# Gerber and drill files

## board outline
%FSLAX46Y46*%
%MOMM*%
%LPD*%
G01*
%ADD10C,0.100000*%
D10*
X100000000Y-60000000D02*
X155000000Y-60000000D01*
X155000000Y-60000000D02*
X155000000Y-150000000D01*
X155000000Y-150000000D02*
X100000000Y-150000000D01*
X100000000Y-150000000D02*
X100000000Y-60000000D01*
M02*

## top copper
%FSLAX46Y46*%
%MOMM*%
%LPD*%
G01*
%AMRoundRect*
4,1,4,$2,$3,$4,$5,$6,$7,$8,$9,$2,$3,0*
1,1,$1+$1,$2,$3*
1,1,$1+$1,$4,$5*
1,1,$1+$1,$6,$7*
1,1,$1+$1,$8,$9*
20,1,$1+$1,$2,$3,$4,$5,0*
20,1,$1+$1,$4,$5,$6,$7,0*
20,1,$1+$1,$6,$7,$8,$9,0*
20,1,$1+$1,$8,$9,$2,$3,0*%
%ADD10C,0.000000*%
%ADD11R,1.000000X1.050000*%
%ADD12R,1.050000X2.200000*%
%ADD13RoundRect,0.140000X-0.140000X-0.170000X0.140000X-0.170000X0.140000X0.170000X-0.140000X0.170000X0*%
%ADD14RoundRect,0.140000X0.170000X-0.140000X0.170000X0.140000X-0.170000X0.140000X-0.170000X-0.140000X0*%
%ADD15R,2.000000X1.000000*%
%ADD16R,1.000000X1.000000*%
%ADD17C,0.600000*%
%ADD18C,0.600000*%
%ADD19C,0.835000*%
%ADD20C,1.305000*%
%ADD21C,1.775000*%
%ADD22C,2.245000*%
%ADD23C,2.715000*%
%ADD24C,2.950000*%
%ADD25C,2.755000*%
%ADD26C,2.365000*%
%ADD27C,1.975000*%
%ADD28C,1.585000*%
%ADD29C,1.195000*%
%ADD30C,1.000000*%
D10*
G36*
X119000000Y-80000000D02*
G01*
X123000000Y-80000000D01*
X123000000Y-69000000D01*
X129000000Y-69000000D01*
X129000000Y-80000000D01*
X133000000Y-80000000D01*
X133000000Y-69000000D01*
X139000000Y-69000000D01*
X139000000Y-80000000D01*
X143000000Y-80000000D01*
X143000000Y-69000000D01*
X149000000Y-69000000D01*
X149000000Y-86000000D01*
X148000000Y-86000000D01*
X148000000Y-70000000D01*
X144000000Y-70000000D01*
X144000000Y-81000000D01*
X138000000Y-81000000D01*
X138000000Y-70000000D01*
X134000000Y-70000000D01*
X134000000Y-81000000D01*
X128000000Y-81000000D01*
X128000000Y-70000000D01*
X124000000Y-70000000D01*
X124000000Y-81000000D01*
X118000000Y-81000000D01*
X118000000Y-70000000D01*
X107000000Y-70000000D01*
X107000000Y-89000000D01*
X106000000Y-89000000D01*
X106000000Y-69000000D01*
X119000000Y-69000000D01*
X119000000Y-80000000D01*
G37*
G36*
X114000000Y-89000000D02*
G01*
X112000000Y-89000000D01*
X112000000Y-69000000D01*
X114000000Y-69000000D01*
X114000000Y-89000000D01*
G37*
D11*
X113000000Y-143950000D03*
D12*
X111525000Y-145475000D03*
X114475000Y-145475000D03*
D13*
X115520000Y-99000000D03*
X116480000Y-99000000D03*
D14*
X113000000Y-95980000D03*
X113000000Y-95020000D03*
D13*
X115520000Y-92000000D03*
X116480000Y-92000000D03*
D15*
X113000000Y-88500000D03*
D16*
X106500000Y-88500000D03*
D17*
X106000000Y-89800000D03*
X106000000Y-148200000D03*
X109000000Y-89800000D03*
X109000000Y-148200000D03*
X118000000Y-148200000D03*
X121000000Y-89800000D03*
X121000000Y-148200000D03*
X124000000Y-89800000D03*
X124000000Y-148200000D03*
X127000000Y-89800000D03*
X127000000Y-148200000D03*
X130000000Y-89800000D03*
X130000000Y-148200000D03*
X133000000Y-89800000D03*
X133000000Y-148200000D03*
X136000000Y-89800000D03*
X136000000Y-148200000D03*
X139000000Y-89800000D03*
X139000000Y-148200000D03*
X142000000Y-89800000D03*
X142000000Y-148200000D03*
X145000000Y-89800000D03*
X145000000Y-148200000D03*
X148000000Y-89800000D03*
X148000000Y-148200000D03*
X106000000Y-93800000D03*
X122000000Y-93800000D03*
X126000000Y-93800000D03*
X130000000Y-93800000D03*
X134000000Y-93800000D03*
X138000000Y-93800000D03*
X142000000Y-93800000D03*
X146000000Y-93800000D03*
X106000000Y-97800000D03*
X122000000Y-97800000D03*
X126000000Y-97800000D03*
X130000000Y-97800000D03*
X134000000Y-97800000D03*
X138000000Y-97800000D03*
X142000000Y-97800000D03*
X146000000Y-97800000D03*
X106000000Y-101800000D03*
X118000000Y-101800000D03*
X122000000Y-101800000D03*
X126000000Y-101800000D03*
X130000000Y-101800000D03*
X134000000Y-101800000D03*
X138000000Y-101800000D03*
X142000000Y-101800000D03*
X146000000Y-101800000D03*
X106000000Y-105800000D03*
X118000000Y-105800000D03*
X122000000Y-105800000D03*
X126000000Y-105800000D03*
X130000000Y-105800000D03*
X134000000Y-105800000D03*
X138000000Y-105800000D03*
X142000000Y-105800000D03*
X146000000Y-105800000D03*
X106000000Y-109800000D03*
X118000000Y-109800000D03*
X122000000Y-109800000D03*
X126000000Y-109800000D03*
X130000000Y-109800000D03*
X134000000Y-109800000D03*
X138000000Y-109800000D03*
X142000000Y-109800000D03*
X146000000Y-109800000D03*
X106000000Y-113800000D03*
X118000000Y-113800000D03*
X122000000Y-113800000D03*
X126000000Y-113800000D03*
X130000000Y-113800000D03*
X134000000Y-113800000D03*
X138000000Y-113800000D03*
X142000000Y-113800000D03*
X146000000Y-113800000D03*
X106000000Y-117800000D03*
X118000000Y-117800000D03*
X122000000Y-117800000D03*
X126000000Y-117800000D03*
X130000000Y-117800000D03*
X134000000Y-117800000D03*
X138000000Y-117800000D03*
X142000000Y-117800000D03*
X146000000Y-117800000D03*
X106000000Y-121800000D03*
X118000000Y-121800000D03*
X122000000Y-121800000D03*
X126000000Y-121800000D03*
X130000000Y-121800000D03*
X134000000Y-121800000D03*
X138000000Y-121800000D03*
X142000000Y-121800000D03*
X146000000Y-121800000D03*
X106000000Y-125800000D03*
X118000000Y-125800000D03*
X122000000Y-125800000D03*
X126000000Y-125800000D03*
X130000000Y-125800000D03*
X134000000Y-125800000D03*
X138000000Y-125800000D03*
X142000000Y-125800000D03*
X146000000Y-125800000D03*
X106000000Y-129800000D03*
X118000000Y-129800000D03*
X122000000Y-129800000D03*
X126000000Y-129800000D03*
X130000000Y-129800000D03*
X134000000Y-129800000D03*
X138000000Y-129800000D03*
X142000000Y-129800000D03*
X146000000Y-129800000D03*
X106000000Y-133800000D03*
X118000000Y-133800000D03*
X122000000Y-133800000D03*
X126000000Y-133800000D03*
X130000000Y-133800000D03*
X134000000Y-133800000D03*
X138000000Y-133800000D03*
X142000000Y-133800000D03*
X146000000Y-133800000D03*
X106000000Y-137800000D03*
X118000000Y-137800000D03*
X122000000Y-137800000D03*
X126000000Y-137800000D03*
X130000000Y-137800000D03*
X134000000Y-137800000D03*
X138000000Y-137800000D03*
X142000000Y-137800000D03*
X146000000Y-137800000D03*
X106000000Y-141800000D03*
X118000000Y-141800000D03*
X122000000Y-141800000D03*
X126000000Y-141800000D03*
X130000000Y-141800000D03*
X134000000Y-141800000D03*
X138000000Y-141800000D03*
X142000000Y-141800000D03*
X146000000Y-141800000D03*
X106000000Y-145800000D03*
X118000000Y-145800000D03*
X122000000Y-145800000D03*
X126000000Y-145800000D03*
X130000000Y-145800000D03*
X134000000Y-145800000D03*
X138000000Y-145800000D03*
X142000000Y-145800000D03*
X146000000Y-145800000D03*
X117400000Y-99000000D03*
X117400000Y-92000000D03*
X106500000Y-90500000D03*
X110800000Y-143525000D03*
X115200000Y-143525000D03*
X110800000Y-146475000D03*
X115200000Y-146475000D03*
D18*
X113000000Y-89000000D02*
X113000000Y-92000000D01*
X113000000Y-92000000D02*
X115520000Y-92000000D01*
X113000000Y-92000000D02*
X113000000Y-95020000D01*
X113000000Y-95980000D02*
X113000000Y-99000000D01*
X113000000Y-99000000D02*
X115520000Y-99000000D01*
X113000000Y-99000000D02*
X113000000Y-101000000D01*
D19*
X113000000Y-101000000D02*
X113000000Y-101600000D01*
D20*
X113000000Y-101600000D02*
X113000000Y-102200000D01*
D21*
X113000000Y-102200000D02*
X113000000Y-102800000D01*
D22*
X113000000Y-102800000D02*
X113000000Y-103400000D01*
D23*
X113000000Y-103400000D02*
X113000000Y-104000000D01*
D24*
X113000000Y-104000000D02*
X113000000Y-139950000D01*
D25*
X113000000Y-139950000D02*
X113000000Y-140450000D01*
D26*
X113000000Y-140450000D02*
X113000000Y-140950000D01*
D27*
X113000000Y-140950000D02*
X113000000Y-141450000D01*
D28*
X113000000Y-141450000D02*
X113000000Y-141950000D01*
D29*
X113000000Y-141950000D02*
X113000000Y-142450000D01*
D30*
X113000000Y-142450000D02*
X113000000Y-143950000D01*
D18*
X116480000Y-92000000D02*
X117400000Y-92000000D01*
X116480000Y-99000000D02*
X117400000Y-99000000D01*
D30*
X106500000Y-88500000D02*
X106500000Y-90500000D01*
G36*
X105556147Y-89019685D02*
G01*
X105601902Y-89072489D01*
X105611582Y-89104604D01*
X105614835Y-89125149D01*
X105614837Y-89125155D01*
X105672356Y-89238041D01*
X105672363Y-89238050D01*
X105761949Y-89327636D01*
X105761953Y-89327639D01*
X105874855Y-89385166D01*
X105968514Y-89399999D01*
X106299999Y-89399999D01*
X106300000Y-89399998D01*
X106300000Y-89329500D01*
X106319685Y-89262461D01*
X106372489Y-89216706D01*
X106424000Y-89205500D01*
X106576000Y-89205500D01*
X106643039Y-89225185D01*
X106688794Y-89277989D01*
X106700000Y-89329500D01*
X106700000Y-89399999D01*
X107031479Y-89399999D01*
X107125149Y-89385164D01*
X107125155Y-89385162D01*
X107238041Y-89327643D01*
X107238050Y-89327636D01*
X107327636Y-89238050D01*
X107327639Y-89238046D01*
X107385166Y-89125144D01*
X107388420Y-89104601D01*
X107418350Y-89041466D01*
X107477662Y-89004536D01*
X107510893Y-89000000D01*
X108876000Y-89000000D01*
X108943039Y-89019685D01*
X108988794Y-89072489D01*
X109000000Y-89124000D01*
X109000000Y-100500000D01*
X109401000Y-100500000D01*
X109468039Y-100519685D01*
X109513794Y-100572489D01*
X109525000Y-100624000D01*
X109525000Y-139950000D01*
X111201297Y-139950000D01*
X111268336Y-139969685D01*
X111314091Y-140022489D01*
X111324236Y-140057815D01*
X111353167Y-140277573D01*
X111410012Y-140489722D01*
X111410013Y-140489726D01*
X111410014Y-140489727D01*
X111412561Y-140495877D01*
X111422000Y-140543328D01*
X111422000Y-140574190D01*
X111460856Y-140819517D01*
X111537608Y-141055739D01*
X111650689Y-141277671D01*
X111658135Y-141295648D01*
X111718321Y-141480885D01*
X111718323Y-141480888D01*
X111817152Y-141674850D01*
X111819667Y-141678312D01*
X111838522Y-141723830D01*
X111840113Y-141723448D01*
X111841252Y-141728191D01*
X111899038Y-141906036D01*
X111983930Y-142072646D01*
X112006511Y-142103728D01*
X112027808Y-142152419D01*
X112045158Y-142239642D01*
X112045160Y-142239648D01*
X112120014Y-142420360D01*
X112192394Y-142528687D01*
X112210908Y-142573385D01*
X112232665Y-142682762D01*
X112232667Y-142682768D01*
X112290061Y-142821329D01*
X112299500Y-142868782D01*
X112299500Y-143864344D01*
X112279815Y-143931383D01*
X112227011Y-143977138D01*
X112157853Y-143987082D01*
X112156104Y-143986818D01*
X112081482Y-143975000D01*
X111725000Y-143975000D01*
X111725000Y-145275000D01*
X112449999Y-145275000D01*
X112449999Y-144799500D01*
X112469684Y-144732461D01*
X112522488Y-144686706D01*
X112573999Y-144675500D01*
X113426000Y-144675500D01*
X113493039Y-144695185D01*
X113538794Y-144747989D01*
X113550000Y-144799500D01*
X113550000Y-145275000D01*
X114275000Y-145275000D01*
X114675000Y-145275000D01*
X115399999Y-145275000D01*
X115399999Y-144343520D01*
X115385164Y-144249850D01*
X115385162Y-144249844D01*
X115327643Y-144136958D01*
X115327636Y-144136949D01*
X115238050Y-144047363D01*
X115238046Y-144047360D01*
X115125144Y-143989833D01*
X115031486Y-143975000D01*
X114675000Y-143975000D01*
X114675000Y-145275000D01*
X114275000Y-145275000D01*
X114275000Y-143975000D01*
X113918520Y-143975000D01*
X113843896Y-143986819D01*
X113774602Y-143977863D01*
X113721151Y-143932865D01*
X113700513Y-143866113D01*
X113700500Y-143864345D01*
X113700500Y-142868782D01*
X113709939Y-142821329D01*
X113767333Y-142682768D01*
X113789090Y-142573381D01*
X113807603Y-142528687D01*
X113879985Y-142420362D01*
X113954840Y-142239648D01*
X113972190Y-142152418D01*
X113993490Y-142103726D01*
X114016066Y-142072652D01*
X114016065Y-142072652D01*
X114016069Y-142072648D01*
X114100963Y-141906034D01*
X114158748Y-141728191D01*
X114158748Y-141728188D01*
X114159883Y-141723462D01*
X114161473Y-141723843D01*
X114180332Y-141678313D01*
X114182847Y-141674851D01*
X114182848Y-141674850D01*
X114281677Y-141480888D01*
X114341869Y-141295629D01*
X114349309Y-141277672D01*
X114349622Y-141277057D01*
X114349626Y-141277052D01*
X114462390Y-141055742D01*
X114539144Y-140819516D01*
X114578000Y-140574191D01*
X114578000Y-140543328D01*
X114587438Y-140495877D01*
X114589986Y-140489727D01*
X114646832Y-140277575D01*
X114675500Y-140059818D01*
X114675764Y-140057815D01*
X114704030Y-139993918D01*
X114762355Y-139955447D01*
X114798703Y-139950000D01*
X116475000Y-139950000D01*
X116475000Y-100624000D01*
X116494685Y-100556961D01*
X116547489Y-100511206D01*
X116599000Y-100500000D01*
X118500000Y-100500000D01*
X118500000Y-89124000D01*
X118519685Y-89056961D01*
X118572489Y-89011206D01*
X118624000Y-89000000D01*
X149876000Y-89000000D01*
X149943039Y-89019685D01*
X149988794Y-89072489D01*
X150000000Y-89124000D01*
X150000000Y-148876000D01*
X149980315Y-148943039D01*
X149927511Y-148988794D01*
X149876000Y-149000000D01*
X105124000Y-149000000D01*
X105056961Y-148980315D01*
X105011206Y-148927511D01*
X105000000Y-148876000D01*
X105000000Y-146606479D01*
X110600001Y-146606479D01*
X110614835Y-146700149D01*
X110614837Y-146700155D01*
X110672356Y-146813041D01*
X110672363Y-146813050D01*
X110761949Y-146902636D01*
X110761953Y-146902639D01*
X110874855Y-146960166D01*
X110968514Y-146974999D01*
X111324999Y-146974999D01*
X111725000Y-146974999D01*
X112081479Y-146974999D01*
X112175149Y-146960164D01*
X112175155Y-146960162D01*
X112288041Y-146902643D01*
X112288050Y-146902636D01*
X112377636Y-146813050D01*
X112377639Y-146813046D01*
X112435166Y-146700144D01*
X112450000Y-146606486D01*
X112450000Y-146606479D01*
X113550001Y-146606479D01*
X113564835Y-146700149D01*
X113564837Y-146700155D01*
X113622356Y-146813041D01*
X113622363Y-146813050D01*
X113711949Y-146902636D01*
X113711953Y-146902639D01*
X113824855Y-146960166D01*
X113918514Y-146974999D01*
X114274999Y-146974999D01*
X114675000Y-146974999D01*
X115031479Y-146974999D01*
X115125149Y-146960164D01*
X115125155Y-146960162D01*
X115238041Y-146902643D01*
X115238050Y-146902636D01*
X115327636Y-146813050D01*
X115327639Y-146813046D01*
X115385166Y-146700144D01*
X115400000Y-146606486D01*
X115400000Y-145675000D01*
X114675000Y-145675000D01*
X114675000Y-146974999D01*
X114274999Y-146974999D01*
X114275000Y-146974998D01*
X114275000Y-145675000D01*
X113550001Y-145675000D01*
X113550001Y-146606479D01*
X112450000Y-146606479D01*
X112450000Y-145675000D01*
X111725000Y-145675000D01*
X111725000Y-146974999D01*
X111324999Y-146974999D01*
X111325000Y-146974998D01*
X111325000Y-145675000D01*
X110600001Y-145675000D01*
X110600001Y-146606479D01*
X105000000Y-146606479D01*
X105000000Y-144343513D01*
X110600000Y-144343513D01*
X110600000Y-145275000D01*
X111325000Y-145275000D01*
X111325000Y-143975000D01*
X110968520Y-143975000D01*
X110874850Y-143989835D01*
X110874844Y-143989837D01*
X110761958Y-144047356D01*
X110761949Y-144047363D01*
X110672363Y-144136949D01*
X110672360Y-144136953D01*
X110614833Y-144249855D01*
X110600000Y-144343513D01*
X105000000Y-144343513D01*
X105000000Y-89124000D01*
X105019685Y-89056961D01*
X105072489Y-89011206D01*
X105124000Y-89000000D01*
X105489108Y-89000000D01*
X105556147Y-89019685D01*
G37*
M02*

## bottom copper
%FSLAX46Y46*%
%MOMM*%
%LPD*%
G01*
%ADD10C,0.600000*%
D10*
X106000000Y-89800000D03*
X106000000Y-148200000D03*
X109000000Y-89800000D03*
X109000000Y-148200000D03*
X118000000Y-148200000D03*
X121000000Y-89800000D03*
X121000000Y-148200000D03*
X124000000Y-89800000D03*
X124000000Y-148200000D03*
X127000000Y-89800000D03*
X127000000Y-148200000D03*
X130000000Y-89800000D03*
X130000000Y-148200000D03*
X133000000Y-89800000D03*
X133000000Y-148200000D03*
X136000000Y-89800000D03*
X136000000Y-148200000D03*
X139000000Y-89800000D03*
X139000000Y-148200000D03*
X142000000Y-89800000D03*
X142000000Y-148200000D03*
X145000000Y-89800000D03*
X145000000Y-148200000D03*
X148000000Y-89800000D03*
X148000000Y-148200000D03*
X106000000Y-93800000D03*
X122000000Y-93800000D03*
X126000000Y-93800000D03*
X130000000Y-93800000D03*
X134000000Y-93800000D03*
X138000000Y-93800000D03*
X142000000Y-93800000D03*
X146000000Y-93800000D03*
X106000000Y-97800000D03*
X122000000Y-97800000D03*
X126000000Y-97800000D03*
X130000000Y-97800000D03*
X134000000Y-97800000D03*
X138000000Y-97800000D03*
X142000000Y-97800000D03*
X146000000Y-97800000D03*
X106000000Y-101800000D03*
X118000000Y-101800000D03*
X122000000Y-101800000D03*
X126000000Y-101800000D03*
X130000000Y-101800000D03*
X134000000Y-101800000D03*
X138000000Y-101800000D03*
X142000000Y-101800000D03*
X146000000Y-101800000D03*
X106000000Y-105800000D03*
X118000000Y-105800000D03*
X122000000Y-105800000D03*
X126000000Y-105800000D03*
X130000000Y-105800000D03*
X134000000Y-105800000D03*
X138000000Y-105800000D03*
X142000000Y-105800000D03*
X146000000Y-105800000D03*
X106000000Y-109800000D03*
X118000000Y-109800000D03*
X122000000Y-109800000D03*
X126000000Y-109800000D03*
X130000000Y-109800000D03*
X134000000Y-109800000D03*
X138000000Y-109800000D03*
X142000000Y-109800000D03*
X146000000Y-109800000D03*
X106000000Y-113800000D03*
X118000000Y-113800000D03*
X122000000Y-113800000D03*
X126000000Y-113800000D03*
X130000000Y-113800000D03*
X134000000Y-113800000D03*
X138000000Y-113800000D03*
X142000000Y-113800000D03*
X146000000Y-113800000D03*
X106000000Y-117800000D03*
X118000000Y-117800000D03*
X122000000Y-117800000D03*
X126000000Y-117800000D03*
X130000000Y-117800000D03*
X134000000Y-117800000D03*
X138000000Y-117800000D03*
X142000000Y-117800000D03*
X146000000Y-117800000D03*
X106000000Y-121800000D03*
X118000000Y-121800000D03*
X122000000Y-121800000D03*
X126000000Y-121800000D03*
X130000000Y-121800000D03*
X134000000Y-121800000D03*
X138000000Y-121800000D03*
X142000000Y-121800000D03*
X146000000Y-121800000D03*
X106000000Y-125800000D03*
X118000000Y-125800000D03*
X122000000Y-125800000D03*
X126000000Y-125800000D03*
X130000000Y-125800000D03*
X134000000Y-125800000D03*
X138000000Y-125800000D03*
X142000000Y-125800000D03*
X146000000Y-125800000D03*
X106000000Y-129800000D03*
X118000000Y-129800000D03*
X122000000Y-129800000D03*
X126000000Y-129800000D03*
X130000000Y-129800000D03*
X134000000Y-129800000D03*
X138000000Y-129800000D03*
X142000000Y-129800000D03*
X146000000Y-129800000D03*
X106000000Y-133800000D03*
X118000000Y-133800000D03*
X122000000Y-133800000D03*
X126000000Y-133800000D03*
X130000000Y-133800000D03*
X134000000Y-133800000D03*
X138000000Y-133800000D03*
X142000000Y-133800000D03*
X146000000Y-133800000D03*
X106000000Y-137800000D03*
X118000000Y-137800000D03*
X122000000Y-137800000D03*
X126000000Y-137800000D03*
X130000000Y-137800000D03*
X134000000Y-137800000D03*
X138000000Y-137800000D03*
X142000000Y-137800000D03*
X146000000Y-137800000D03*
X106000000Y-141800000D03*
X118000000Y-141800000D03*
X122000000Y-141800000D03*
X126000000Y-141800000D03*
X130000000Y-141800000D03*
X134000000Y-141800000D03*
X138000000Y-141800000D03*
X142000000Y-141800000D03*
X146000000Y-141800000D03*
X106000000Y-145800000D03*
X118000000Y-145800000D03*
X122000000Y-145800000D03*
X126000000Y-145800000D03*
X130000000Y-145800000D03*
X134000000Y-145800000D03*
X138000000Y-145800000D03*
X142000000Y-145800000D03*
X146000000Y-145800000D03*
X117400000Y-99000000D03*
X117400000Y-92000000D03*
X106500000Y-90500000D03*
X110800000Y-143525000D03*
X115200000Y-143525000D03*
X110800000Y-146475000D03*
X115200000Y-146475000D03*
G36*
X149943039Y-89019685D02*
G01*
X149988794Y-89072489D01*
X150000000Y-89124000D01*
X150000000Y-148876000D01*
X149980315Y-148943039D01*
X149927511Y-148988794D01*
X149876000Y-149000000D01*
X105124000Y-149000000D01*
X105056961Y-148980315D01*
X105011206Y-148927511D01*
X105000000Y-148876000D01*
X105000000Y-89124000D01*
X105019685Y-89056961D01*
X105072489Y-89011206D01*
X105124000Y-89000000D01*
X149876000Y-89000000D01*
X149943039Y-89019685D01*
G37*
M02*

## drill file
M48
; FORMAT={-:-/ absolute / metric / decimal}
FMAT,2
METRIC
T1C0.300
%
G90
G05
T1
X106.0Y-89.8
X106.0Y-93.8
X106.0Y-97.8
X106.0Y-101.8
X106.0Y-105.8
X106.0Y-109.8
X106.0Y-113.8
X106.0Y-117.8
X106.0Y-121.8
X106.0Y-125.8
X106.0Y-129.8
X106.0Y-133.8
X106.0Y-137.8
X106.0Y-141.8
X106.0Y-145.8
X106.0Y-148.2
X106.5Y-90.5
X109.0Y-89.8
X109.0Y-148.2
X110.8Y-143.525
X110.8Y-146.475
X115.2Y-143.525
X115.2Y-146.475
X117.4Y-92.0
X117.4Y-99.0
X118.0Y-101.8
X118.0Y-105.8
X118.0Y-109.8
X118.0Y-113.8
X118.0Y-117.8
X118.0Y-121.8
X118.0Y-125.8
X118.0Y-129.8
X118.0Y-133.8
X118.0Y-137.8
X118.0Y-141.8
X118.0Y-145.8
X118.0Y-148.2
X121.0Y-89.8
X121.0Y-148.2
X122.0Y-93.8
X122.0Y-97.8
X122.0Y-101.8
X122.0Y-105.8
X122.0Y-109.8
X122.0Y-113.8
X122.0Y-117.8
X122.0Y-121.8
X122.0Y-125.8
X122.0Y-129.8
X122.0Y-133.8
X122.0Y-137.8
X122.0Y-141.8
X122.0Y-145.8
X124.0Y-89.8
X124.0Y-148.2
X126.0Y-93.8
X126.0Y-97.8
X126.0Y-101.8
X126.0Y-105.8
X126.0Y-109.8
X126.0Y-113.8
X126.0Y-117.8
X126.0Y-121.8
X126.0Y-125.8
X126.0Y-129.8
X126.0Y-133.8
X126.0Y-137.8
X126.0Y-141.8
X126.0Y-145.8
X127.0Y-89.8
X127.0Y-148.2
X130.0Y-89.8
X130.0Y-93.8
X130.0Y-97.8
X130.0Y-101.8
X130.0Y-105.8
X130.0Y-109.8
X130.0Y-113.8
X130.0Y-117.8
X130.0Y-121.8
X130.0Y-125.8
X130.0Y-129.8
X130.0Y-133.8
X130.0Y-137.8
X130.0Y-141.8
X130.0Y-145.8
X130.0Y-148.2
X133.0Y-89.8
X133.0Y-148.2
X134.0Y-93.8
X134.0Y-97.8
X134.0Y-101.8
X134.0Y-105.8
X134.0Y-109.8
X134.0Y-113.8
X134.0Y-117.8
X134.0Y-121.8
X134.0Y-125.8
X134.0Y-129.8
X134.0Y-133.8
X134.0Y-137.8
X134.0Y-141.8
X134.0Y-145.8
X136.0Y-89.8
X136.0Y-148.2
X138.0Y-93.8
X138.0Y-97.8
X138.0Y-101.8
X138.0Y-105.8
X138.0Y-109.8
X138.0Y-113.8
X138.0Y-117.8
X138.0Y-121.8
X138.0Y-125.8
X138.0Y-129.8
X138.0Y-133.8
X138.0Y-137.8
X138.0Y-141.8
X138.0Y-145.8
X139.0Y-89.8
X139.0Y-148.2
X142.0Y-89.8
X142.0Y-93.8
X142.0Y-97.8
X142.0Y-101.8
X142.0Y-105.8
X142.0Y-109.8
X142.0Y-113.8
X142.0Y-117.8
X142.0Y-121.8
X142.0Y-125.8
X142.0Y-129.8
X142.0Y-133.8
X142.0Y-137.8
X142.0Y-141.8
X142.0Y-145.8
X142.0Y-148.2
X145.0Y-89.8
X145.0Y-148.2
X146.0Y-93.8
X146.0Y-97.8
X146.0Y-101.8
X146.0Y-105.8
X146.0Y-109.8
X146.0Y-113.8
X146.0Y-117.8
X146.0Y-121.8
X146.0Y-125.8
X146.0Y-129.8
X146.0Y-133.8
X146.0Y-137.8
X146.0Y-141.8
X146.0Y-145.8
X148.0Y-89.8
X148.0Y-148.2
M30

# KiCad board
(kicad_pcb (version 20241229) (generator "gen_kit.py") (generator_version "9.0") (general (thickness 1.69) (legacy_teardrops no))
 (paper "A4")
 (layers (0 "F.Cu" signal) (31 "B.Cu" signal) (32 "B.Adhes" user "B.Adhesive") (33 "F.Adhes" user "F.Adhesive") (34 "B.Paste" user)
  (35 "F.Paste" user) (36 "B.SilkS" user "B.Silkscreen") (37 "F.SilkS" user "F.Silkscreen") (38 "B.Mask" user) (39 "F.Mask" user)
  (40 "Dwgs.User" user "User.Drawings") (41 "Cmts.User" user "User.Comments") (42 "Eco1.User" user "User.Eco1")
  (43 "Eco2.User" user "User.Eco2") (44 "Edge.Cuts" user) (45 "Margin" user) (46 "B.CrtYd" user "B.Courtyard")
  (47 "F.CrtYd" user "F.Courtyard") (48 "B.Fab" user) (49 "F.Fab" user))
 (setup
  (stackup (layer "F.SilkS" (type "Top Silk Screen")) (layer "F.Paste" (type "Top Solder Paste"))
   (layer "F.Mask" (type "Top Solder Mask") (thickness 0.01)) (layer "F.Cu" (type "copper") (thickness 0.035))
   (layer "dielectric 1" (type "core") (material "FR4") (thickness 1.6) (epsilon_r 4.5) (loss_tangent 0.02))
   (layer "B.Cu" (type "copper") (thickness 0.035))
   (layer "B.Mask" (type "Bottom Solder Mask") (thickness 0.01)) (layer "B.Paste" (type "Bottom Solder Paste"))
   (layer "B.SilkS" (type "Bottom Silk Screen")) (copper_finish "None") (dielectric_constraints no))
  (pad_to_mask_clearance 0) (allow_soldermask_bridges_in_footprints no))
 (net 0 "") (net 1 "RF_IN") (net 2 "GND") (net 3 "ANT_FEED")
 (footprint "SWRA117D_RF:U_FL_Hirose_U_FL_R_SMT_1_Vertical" (layer "F.Cu") (at 113 145 270)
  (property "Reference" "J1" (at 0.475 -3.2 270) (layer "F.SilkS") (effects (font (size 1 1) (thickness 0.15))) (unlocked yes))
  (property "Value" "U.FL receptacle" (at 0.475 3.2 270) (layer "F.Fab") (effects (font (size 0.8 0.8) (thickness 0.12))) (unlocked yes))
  (pad "1" smd rect (at -1.05 0 270) (size 1.05 1) (layers "F.Cu" "F.Paste" "F.Mask") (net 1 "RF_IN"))
  (pad "2" smd rect (at 0.475 1.475 270) (size 2.2 1.05) (layers "F.Cu" "F.Paste" "F.Mask") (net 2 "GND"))
  (pad "2" smd rect (at 0.475 -1.475 270) (size 2.2 1.05) (layers "F.Cu" "F.Paste" "F.Mask") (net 2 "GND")))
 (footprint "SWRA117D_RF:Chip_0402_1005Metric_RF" (layer "F.Cu") (at 116 99)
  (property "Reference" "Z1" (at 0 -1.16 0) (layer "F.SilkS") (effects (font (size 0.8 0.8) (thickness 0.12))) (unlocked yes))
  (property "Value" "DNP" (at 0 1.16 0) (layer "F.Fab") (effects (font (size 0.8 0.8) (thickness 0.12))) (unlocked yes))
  (pad "1" smd roundrect (at -0.48 0) (size 0.56 0.62) (layers "F.Cu" "F.Paste" "F.Mask") (roundrect_rratio 0.25) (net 1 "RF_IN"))
  (pad "2" smd roundrect (at 0.48 0) (size 0.56 0.62) (layers "F.Cu" "F.Paste" "F.Mask") (roundrect_rratio 0.25) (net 2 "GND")))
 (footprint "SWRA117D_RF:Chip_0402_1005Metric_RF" (layer "F.Cu") (at 113 95.5 90)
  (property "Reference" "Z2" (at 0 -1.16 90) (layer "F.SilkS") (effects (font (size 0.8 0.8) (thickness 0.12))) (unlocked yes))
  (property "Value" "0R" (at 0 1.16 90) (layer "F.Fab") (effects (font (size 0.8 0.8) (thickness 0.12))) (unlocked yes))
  (pad "1" smd roundrect (at -0.48 0 90) (size 0.56 0.62) (layers "F.Cu" "F.Paste" "F.Mask") (roundrect_rratio 0.25) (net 1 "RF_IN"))
  (pad "2" smd roundrect (at 0.48 0 90) (size 0.56 0.62) (layers "F.Cu" "F.Paste" "F.Mask") (roundrect_rratio 0.25) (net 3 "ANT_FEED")))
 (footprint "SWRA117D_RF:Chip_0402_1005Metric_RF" (layer "F.Cu") (at 116 92)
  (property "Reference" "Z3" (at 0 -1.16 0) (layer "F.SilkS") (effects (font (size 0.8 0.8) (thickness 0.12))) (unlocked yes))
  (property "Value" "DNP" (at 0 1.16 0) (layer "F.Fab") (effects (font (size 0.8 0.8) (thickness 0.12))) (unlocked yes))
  (pad "1" smd roundrect (at -0.48 0) (size 0.56 0.62) (layers "F.Cu" "F.Paste" "F.Mask") (roundrect_rratio 0.25) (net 3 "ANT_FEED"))
  (pad "2" smd roundrect (at 0.48 0) (size 0.56 0.62) (layers "F.Cu" "F.Paste" "F.Mask") (roundrect_rratio 0.25) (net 2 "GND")))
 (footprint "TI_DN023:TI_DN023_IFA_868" (layer "F.Cu") (at 113 89)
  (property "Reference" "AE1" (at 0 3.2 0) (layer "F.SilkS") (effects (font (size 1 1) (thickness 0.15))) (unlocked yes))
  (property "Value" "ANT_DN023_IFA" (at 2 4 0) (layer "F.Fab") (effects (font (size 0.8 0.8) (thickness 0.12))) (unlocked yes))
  (fp_poly
   (pts (xy -6 0) (xy -6 -19) (xy 5 -19) (xy 5 -8) (xy 11 -8) (xy 11 -19) (xy 15 -19) (xy 15 -8) (xy 21 -8) (xy 21 -19) (xy 25 -19)
    (xy 25 -8) (xy 31 -8) (xy 31 -19) (xy 35 -19) (xy 35 -3) (xy 36 -3) (xy 36 -20) (xy 30 -20) (xy 30 -9) (xy 26 -9) (xy 26 -20)
    (xy 20 -20) (xy 20 -9) (xy 16 -9) (xy 16 -20) (xy 10 -20) (xy 10 -9) (xy 6 -9) (xy 6 -20) (xy -7 -20) (xy -7 0))
   (stroke (width 0) (type solid)) (fill yes) (layer "F.Cu"))
  (fp_poly (pts (xy 1 0) (xy 1 -20) (xy -1 -20) (xy -1 0)) (stroke (width 0) (type solid)) (fill yes) (layer "F.Cu"))
  (pad "1" smd rect (at 0 -0.5) (size 2 1) (layers "F.Cu" "F.Mask") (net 3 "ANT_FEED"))
  (pad "2" smd rect (at -6.5 -0.5) (size 1 1) (layers "F.Cu" "F.Mask") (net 2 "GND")))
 (gr_line (start 100 60) (end 155 60) (stroke (width 0.1) (type solid)) (layer "Edge.Cuts"))
 (gr_line (start 155 60) (end 155 150) (stroke (width 0.1) (type solid)) (layer "Edge.Cuts"))
 (gr_line (start 155 150) (end 100 150) (stroke (width 0.1) (type solid)) (layer "Edge.Cuts"))
 (gr_line (start 100 150) (end 100 60) (stroke (width 0.1) (type solid)) (layer "Edge.Cuts"))
 (segment (start 113 89) (end 113 92) (width 0.6) (layer "F.Cu") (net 3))
 (segment (start 113 92) (end 115.52 92) (width 0.6) (layer "F.Cu") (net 3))
 (segment (start 113 92) (end 113 95.02) (width 0.6) (layer "F.Cu") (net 3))
 (segment (start 113 95.98) (end 113 99) (width 0.6) (layer "F.Cu") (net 1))
 (segment (start 113 99) (end 115.52 99) (width 0.6) (layer "F.Cu") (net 1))
 (segment (start 113 99) (end 113 101) (width 0.6) (layer "F.Cu") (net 1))
 (segment (start 113 101) (end 113 101.6) (width 0.835) (layer "F.Cu") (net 1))
 (segment (start 113 101.6) (end 113 102.2) (width 1.305) (layer "F.Cu") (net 1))
 (segment (start 113 102.2) (end 113 102.8) (width 1.775) (layer "F.Cu") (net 1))
 (segment (start 113 102.8) (end 113 103.4) (width 2.245) (layer "F.Cu") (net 1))
 (segment (start 113 103.4) (end 113 104) (width 2.715) (layer "F.Cu") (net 1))
 (segment (start 113 104) (end 113 139.95) (width 2.95) (layer "F.Cu") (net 1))
 (segment (start 113 139.95) (end 113 140.45) (width 2.755) (layer "F.Cu") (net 1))
 (segment (start 113 140.45) (end 113 140.95) (width 2.365) (layer "F.Cu") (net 1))
 (segment (start 113 140.95) (end 113 141.45) (width 1.975) (layer "F.Cu") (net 1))
 (segment (start 113 141.45) (end 113 141.95) (width 1.585) (layer "F.Cu") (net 1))
 (segment (start 113 141.95) (end 113 142.45) (width 1.195) (layer "F.Cu") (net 1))
 (segment (start 113 142.45) (end 113 143.95) (width 1) (layer "F.Cu") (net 1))
 (segment (start 116.48 92) (end 117.4 92) (width 0.6) (layer "F.Cu") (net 2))
 (segment (start 116.48 99) (end 117.4 99) (width 0.6) (layer "F.Cu") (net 2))
 (segment (start 106.5 88.5) (end 106.5 90.5) (width 1) (layer "F.Cu") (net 2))
 (via (at 106 89.8) (size 0.6) (drill 0.3) (layers "F.Cu" "B.Cu") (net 2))
 (via (at 106 148.2) (size 0.6) (drill 0.3) (layers "F.Cu" "B.Cu") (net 2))
 (via (at 109 89.8) (size 0.6) (drill 0.3) (layers "F.Cu" "B.Cu") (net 2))
 (via (at 109 148.2) (size 0.6) (drill 0.3) (layers "F.Cu" "B.Cu") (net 2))
 (via (at 118 148.2) (size 0.6) (drill 0.3) (layers "F.Cu" "B.Cu") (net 2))
 (via (at 121 89.8) (size 0.6) (drill 0.3) (layers "F.Cu" "B.Cu") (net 2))
 (via (at 121 148.2) (size 0.6) (drill 0.3) (layers "F.Cu" "B.Cu") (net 2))
 (via (at 124 89.8) (size 0.6) (drill 0.3) (layers "F.Cu" "B.Cu") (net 2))
 (via (at 124 148.2) (size 0.6) (drill 0.3) (layers "F.Cu" "B.Cu") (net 2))
 (via (at 127 89.8) (size 0.6) (drill 0.3) (layers "F.Cu" "B.Cu") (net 2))
 (via (at 127 148.2) (size 0.6) (drill 0.3) (layers "F.Cu" "B.Cu") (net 2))
 (via (at 130 89.8) (size 0.6) (drill 0.3) (layers "F.Cu" "B.Cu") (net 2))
 (via (at 130 148.2) (size 0.6) (drill 0.3) (layers "F.Cu" "B.Cu") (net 2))
 (via (at 133 89.8) (size 0.6) (drill 0.3) (layers "F.Cu" "B.Cu") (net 2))
 (via (at 133 148.2) (size 0.6) (drill 0.3) (layers "F.Cu" "B.Cu") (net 2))
 (via (at 136 89.8) (size 0.6) (drill 0.3) (layers "F.Cu" "B.Cu") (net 2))
 (via (at 136 148.2) (size 0.6) (drill 0.3) (layers "F.Cu" "B.Cu") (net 2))
 (via (at 139 89.8) (size 0.6) (drill 0.3) (layers "F.Cu" "B.Cu") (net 2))
 (via (at 139 148.2) (size 0.6) (drill 0.3) (layers "F.Cu" "B.Cu") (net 2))
 (via (at 142 89.8) (size 0.6) (drill 0.3) (layers "F.Cu" "B.Cu") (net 2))
 (via (at 142 148.2) (size 0.6) (drill 0.3) (layers "F.Cu" "B.Cu") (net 2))
 (via (at 145 89.8) (size 0.6) (drill 0.3) (layers "F.Cu" "B.Cu") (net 2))
 (via (at 145 148.2) (size 0.6) (drill 0.3) (layers "F.Cu" "B.Cu") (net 2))
 (via (at 148 89.8) (size 0.6) (drill 0.3) (layers "F.Cu" "B.Cu") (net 2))
 (via (at 148 148.2) (size 0.6) (drill 0.3) (layers "F.Cu" "B.Cu") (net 2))
 (via (at 106 93.8) (size 0.6) (drill 0.3) (layers "F.Cu" "B.Cu") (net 2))
 (via (at 122 93.8) (size 0.6) (drill 0.3) (layers "F.Cu" "B.Cu") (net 2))
 (via (at 126 93.8) (size 0.6) (drill 0.3) (layers "F.Cu" "B.Cu") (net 2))
 (via (at 130 93.8) (size 0.6) (drill 0.3) (layers "F.Cu" "B.Cu") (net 2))
 (via (at 134 93.8) (size 0.6) (drill 0.3) (layers "F.Cu" "B.Cu") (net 2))
 (via (at 138 93.8) (size 0.6) (drill 0.3) (layers "F.Cu" "B.Cu") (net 2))
 (via (at 142 93.8) (size 0.6) (drill 0.3) (layers "F.Cu" "B.Cu") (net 2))
 (via (at 146 93.8) (size 0.6) (drill 0.3) (layers "F.Cu" "B.Cu") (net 2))
 (via (at 106 97.8) (size 0.6) (drill 0.3) (layers "F.Cu" "B.Cu") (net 2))
 (via (at 122 97.8) (size 0.6) (drill 0.3) (layers "F.Cu" "B.Cu") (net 2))
 (via (at 126 97.8) (size 0.6) (drill 0.3) (layers "F.Cu" "B.Cu") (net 2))
 (via (at 130 97.8) (size 0.6) (drill 0.3) (layers "F.Cu" "B.Cu") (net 2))
 (via (at 134 97.8) (size 0.6) (drill 0.3) (layers "F.Cu" "B.Cu") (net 2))
 (via (at 138 97.8) (size 0.6) (drill 0.3) (layers "F.Cu" "B.Cu") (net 2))
 (via (at 142 97.8) (size 0.6) (drill 0.3) (layers "F.Cu" "B.Cu") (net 2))
 (via (at 146 97.8) (size 0.6) (drill 0.3) (layers "F.Cu" "B.Cu") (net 2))
 (via (at 106 101.8) (size 0.6) (drill 0.3) (layers "F.Cu" "B.Cu") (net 2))
 (via (at 118 101.8) (size 0.6) (drill 0.3) (layers "F.Cu" "B.Cu") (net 2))
 (via (at 122 101.8) (size 0.6) (drill 0.3) (layers "F.Cu" "B.Cu") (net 2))
 (via (at 126 101.8) (size 0.6) (drill 0.3) (layers "F.Cu" "B.Cu") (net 2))
 (via (at 130 101.8) (size 0.6) (drill 0.3) (layers "F.Cu" "B.Cu") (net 2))
 (via (at 134 101.8) (size 0.6) (drill 0.3) (layers "F.Cu" "B.Cu") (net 2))
 (via (at 138 101.8) (size 0.6) (drill 0.3) (layers "F.Cu" "B.Cu") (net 2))
 (via (at 142 101.8) (size 0.6) (drill 0.3) (layers "F.Cu" "B.Cu") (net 2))
 (via (at 146 101.8) (size 0.6) (drill 0.3) (layers "F.Cu" "B.Cu") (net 2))
 (via (at 106 105.8) (size 0.6) (drill 0.3) (layers "F.Cu" "B.Cu") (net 2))
 (via (at 118 105.8) (size 0.6) (drill 0.3) (layers "F.Cu" "B.Cu") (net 2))
 (via (at 122 105.8) (size 0.6) (drill 0.3) (layers "F.Cu" "B.Cu") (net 2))
 (via (at 126 105.8) (size 0.6) (drill 0.3) (layers "F.Cu" "B.Cu") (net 2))
 (via (at 130 105.8) (size 0.6) (drill 0.3) (layers "F.Cu" "B.Cu") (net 2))
 (via (at 134 105.8) (size 0.6) (drill 0.3) (layers "F.Cu" "B.Cu") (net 2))
 (via (at 138 105.8) (size 0.6) (drill 0.3) (layers "F.Cu" "B.Cu") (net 2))
 (via (at 142 105.8) (size 0.6) (drill 0.3) (layers "F.Cu" "B.Cu") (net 2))
 (via (at 146 105.8) (size 0.6) (drill 0.3) (layers "F.Cu" "B.Cu") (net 2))
 (via (at 106 109.8) (size 0.6) (drill 0.3) (layers "F.Cu" "B.Cu") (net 2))
 (via (at 118 109.8) (size 0.6) (drill 0.3) (layers "F.Cu" "B.Cu") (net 2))
 (via (at 122 109.8) (size 0.6) (drill 0.3) (layers "F.Cu" "B.Cu") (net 2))
 (via (at 126 109.8) (size 0.6) (drill 0.3) (layers "F.Cu" "B.Cu") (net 2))
 (via (at 130 109.8) (size 0.6) (drill 0.3) (layers "F.Cu" "B.Cu") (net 2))
 (via (at 134 109.8) (size 0.6) (drill 0.3) (layers "F.Cu" "B.Cu") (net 2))
 (via (at 138 109.8) (size 0.6) (drill 0.3) (layers "F.Cu" "B.Cu") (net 2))
 (via (at 142 109.8) (size 0.6) (drill 0.3) (layers "F.Cu" "B.Cu") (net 2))
 (via (at 146 109.8) (size 0.6) (drill 0.3) (layers "F.Cu" "B.Cu") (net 2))
 (via (at 106 113.8) (size 0.6) (drill 0.3) (layers "F.Cu" "B.Cu") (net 2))
 (via (at 118 113.8) (size 0.6) (drill 0.3) (layers "F.Cu" "B.Cu") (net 2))
 (via (at 122 113.8) (size 0.6) (drill 0.3) (layers "F.Cu" "B.Cu") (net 2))
 (via (at 126 113.8) (size 0.6) (drill 0.3) (layers "F.Cu" "B.Cu") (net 2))
 (via (at 130 113.8) (size 0.6) (drill 0.3) (layers "F.Cu" "B.Cu") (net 2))
 (via (at 134 113.8) (size 0.6) (drill 0.3) (layers "F.Cu" "B.Cu") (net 2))
 (via (at 138 113.8) (size 0.6) (drill 0.3) (layers "F.Cu" "B.Cu") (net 2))
 (via (at 142 113.8) (size 0.6) (drill 0.3) (layers "F.Cu" "B.Cu") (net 2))
 (via (at 146 113.8) (size 0.6) (drill 0.3) (layers "F.Cu" "B.Cu") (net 2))
 (via (at 106 117.8) (size 0.6) (drill 0.3) (layers "F.Cu" "B.Cu") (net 2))
 (via (at 118 117.8) (size 0.6) (drill 0.3) (layers "F.Cu" "B.Cu") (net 2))
 (via (at 122 117.8) (size 0.6) (drill 0.3) (layers "F.Cu" "B.Cu") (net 2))
 (via (at 126 117.8) (size 0.6) (drill 0.3) (layers "F.Cu" "B.Cu") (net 2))
 (via (at 130 117.8) (size 0.6) (drill 0.3) (layers "F.Cu" "B.Cu") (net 2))
 (via (at 134 117.8) (size 0.6) (drill 0.3) (layers "F.Cu" "B.Cu") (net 2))
 (via (at 138 117.8) (size 0.6) (drill 0.3) (layers "F.Cu" "B.Cu") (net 2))
 (via (at 142 117.8) (size 0.6) (drill 0.3) (layers "F.Cu" "B.Cu") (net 2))
 (via (at 146 117.8) (size 0.6) (drill 0.3) (layers "F.Cu" "B.Cu") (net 2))
 (via (at 106 121.8) (size 0.6) (drill 0.3) (layers "F.Cu" "B.Cu") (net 2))
 (via (at 118 121.8) (size 0.6) (drill 0.3) (layers "F.Cu" "B.Cu") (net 2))
 (via (at 122 121.8) (size 0.6) (drill 0.3) (layers "F.Cu" "B.Cu") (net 2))
 (via (at 126 121.8) (size 0.6) (drill 0.3) (layers "F.Cu" "B.Cu") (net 2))
 (via (at 130 121.8) (size 0.6) (drill 0.3) (layers "F.Cu" "B.Cu") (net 2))
 (via (at 134 121.8) (size 0.6) (drill 0.3) (layers "F.Cu" "B.Cu") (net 2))
 (via (at 138 121.8) (size 0.6) (drill 0.3) (layers "F.Cu" "B.Cu") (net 2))
 (via (at 142 121.8) (size 0.6) (drill 0.3) (layers "F.Cu" "B.Cu") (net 2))
 (via (at 146 121.8) (size 0.6) (drill 0.3) (layers "F.Cu" "B.Cu") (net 2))
 (via (at 106 125.8) (size 0.6) (drill 0.3) (layers "F.Cu" "B.Cu") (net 2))
 (via (at 118 125.8) (size 0.6) (drill 0.3) (layers "F.Cu" "B.Cu") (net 2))
 (via (at 122 125.8) (size 0.6) (drill 0.3) (layers "F.Cu" "B.Cu") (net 2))
 (via (at 126 125.8) (size 0.6) (drill 0.3) (layers "F.Cu" "B.Cu") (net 2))
 (via (at 130 125.8) (size 0.6) (drill 0.3) (layers "F.Cu" "B.Cu") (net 2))
 (via (at 134 125.8) (size 0.6) (drill 0.3) (layers "F.Cu" "B.Cu") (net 2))
 (via (at 138 125.8) (size 0.6) (drill 0.3) (layers "F.Cu" "B.Cu") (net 2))
 (via (at 142 125.8) (size 0.6) (drill 0.3) (layers "F.Cu" "B.Cu") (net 2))
 (via (at 146 125.8) (size 0.6) (drill 0.3) (layers "F.Cu" "B.Cu") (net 2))
 (via (at 106 129.8) (size 0.6) (drill 0.3) (layers "F.Cu" "B.Cu") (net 2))
 (via (at 118 129.8) (size 0.6) (drill 0.3) (layers "F.Cu" "B.Cu") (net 2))
 (via (at 122 129.8) (size 0.6) (drill 0.3) (layers "F.Cu" "B.Cu") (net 2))
 (via (at 126 129.8) (size 0.6) (drill 0.3) (layers "F.Cu" "B.Cu") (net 2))
 (via (at 130 129.8) (size 0.6) (drill 0.3) (layers "F.Cu" "B.Cu") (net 2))
 (via (at 134 129.8) (size 0.6) (drill 0.3) (layers "F.Cu" "B.Cu") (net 2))
 (via (at 138 129.8) (size 0.6) (drill 0.3) (layers "F.Cu" "B.Cu") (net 2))
 (via (at 142 129.8) (size 0.6) (drill 0.3) (layers "F.Cu" "B.Cu") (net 2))
 (via (at 146 129.8) (size 0.6) (drill 0.3) (layers "F.Cu" "B.Cu") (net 2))
 (via (at 106 133.8) (size 0.6) (drill 0.3) (layers "F.Cu" "B.Cu") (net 2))
 (via (at 118 133.8) (size 0.6) (drill 0.3) (layers "F.Cu" "B.Cu") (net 2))
 (via (at 122 133.8) (size 0.6) (drill 0.3) (layers "F.Cu" "B.Cu") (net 2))
 (via (at 126 133.8) (size 0.6) (drill 0.3) (layers "F.Cu" "B.Cu") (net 2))
 (via (at 130 133.8) (size 0.6) (drill 0.3) (layers "F.Cu" "B.Cu") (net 2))
 (via (at 134 133.8) (size 0.6) (drill 0.3) (layers "F.Cu" "B.Cu") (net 2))
 (via (at 138 133.8) (size 0.6) (drill 0.3) (layers "F.Cu" "B.Cu") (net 2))
 (via (at 142 133.8) (size 0.6) (drill 0.3) (layers "F.Cu" "B.Cu") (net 2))
 (via (at 146 133.8) (size 0.6) (drill 0.3) (layers "F.Cu" "B.Cu") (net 2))
 (via (at 106 137.8) (size 0.6) (drill 0.3) (layers "F.Cu" "B.Cu") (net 2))
 (via (at 118 137.8) (size 0.6) (drill 0.3) (layers "F.Cu" "B.Cu") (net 2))
 (via (at 122 137.8) (size 0.6) (drill 0.3) (layers "F.Cu" "B.Cu") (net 2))
 (via (at 126 137.8) (size 0.6) (drill 0.3) (layers "F.Cu" "B.Cu") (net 2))
 (via (at 130 137.8) (size 0.6) (drill 0.3) (layers "F.Cu" "B.Cu") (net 2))
 (via (at 134 137.8) (size 0.6) (drill 0.3) (layers "F.Cu" "B.Cu") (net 2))
 (via (at 138 137.8) (size 0.6) (drill 0.3) (layers "F.Cu" "B.Cu") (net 2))
 (via (at 142 137.8) (size 0.6) (drill 0.3) (layers "F.Cu" "B.Cu") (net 2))
 (via (at 146 137.8) (size 0.6) (drill 0.3) (layers "F.Cu" "B.Cu") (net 2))
 (via (at 106 141.8) (size 0.6) (drill 0.3) (layers "F.Cu" "B.Cu") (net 2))
 (via (at 118 141.8) (size 0.6) (drill 0.3) (layers "F.Cu" "B.Cu") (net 2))
 (via (at 122 141.8) (size 0.6) (drill 0.3) (layers "F.Cu" "B.Cu") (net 2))
 (via (at 126 141.8) (size 0.6) (drill 0.3) (layers "F.Cu" "B.Cu") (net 2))
 (via (at 130 141.8) (size 0.6) (drill 0.3) (layers "F.Cu" "B.Cu") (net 2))
 (via (at 134 141.8) (size 0.6) (drill 0.3) (layers "F.Cu" "B.Cu") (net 2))
 (via (at 138 141.8) (size 0.6) (drill 0.3) (layers "F.Cu" "B.Cu") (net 2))
 (via (at 142 141.8) (size 0.6) (drill 0.3) (layers "F.Cu" "B.Cu") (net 2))
 (via (at 146 141.8) (size 0.6) (drill 0.3) (layers "F.Cu" "B.Cu") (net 2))
 (via (at 106 145.8) (size 0.6) (drill 0.3) (layers "F.Cu" "B.Cu") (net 2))
 (via (at 118 145.8) (size 0.6) (drill 0.3) (layers "F.Cu" "B.Cu") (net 2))
 (via (at 122 145.8) (size 0.6) (drill 0.3) (layers "F.Cu" "B.Cu") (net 2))
 (via (at 126 145.8) (size 0.6) (drill 0.3) (layers "F.Cu" "B.Cu") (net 2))
 (via (at 130 145.8) (size 0.6) (drill 0.3) (layers "F.Cu" "B.Cu") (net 2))
 (via (at 134 145.8) (size 0.6) (drill 0.3) (layers "F.Cu" "B.Cu") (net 2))
 (via (at 138 145.8) (size 0.6) (drill 0.3) (layers "F.Cu" "B.Cu") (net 2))
 (via (at 142 145.8) (size 0.6) (drill 0.3) (layers "F.Cu" "B.Cu") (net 2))
 (via (at 146 145.8) (size 0.6) (drill 0.3) (layers "F.Cu" "B.Cu") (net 2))
 (via (at 117.4 99) (size 0.6) (drill 0.3) (layers "F.Cu" "B.Cu") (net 2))
 (via (at 117.4 92) (size 0.6) (drill 0.3) (layers "F.Cu" "B.Cu") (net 2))
 (via (at 106.5 90.5) (size 0.6) (drill 0.3) (layers "F.Cu" "B.Cu") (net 2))
 (via (at 110.8 143.525) (size 0.6) (drill 0.3) (layers "F.Cu" "B.Cu") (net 2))
 (via (at 115.2 143.525) (size 0.6) (drill 0.3) (layers "F.Cu" "B.Cu") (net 2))
 (via (at 110.8 146.475) (size 0.6) (drill 0.3) (layers "F.Cu" "B.Cu") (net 2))
 (via (at 115.2 146.475) (size 0.6) (drill 0.3) (layers "F.Cu" "B.Cu") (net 2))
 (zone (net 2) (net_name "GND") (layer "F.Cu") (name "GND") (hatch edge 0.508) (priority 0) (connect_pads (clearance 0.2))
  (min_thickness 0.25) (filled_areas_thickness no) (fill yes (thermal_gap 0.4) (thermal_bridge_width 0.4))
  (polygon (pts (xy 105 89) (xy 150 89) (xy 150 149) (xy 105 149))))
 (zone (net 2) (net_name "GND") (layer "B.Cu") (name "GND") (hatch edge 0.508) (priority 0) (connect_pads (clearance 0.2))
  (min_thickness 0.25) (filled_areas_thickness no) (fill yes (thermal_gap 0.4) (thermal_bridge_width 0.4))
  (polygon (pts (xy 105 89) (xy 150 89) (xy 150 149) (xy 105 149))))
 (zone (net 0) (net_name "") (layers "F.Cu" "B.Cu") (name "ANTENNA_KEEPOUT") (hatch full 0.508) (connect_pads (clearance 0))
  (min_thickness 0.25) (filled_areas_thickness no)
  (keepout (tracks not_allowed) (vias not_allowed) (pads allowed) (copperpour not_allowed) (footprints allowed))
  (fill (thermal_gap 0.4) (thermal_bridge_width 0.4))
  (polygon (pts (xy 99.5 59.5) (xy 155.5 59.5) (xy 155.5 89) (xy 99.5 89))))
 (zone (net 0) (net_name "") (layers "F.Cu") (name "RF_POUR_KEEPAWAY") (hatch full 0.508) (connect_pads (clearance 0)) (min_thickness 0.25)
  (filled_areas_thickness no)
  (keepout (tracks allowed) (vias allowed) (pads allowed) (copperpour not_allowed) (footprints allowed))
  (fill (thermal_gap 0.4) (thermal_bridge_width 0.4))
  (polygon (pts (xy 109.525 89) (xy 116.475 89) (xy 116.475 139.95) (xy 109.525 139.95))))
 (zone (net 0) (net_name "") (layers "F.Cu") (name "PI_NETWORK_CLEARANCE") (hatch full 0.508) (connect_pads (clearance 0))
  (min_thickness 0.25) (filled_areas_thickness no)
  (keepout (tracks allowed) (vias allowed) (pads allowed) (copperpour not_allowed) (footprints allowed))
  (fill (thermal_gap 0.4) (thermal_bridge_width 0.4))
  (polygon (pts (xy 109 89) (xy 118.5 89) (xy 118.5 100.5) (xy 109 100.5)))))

